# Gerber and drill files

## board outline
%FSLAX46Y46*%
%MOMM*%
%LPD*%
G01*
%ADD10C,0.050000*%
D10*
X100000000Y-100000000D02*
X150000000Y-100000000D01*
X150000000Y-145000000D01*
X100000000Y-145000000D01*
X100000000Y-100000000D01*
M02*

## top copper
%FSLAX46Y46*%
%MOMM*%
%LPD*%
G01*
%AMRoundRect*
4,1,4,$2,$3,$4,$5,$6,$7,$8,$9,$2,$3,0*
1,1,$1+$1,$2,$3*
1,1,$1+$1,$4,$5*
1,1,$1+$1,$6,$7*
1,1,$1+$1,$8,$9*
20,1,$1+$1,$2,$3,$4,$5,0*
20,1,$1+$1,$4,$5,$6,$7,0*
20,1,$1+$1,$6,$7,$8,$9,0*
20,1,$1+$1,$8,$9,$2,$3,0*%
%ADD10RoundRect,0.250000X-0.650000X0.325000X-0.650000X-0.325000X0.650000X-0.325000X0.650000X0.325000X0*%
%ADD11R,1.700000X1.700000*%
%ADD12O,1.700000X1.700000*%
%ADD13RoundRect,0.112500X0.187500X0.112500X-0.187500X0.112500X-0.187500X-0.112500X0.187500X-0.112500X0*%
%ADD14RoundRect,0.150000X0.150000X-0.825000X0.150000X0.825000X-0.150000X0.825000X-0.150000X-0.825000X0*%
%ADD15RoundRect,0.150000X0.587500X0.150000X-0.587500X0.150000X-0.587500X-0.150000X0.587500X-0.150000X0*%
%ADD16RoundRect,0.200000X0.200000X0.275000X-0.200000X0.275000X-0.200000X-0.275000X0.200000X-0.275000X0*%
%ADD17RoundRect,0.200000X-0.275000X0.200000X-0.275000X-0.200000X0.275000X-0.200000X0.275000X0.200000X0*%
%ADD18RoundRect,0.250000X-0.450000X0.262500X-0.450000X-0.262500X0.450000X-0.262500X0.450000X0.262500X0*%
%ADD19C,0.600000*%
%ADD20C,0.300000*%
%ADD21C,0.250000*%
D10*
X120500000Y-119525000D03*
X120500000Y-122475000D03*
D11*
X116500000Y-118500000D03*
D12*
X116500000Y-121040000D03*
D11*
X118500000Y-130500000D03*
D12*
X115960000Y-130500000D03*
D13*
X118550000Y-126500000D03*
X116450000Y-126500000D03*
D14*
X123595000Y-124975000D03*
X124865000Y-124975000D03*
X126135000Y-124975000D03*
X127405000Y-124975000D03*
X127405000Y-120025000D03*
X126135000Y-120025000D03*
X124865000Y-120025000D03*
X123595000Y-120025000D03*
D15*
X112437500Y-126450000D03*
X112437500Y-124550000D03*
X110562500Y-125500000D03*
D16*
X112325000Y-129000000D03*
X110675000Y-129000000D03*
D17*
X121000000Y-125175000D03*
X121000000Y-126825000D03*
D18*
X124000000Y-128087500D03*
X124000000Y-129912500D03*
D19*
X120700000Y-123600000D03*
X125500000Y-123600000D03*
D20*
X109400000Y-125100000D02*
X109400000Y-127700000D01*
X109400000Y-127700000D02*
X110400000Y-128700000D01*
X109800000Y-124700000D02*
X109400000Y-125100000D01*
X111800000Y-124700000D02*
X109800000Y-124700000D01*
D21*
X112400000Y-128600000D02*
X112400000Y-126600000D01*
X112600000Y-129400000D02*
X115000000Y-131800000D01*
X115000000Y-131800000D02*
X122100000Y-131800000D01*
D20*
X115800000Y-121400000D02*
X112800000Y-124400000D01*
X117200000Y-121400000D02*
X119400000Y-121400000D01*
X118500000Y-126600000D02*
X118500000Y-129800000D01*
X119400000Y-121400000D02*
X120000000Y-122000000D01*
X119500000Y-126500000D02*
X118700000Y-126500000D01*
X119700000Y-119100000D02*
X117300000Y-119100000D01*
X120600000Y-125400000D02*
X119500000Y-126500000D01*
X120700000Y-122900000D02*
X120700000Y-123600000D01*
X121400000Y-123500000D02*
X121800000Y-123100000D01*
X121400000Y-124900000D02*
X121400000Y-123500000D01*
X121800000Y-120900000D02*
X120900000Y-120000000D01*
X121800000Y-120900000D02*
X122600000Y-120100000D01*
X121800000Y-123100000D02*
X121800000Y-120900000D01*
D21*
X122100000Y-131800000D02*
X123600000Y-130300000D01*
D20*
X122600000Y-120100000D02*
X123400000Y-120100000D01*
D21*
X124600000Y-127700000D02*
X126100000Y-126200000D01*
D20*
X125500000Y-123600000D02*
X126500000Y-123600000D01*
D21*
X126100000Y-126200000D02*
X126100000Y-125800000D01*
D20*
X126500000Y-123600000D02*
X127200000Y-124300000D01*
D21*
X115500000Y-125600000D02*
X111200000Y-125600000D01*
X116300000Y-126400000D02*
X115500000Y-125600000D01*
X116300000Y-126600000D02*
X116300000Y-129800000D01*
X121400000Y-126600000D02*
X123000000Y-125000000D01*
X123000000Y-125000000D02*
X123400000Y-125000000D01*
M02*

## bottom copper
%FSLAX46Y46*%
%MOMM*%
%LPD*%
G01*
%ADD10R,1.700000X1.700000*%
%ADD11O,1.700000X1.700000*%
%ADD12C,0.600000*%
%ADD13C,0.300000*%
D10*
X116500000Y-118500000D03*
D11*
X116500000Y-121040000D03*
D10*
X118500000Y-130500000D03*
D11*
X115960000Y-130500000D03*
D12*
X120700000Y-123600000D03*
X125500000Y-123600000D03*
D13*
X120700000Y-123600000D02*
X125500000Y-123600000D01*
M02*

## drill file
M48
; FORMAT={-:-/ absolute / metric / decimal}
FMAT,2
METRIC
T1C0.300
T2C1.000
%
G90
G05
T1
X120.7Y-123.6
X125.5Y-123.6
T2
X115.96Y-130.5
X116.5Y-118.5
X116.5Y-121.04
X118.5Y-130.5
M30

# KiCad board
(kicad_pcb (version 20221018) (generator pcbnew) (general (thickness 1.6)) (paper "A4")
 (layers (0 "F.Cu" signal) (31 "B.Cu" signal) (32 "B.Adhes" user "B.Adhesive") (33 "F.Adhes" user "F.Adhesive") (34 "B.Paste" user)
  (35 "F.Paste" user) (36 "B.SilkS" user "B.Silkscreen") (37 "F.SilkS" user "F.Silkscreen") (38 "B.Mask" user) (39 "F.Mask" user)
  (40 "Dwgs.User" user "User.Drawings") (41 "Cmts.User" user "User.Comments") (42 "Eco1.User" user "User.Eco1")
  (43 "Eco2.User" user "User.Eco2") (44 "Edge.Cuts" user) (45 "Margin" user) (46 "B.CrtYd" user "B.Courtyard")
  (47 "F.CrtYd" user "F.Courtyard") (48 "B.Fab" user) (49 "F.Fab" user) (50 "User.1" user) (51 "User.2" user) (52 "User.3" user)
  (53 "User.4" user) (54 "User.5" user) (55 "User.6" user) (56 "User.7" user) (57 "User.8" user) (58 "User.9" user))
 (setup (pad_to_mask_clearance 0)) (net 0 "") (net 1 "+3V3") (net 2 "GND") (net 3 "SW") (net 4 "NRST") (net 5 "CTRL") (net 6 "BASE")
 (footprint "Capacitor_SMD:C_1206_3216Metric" (layer "F.Cu") (at 120.5 121 -90)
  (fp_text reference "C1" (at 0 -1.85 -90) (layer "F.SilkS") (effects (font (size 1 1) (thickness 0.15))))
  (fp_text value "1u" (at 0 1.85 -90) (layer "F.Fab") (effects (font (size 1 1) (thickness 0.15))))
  (pad "1" smd roundrect (at -1.475 0 270) (size 1.15 1.8) (layers "F.Cu" "F.Paste" "F.Mask") (roundrect_rratio 0.217391) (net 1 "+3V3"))
  (pad "2" smd roundrect (at 1.475 0 270) (size 1.15 1.8) (layers "F.Cu" "F.Paste" "F.Mask") (roundrect_rratio 0.217391) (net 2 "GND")))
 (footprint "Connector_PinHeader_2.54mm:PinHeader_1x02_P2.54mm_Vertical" (layer "F.Cu") (at 116.5 118.5)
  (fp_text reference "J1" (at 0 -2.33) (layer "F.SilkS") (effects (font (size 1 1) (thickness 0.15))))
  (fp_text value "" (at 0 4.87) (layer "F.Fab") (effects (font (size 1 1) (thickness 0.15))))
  (pad "1" thru_hole rect (at 0 0) (size 1.7 1.7) (drill 1) (layers "*.Cu" "*.Mask") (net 1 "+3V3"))
  (pad "2" thru_hole oval (at 0 2.54) (size 1.7 1.7) (drill 1) (layers "*.Cu" "*.Mask") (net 2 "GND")))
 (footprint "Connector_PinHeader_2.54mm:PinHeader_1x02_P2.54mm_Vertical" (layer "F.Cu") (at 118.5 130.5 -90)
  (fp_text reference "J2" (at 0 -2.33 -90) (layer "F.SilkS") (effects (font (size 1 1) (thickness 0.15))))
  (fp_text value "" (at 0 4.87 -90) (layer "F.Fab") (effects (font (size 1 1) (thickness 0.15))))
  (pad "1" thru_hole rect (at 0 0 270) (size 1.7 1.7) (drill 1) (layers "*.Cu" "*.Mask") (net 1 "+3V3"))
  (pad "2" thru_hole oval (at 0 2.54 270) (size 1.7 1.7) (drill 1) (layers "*.Cu" "*.Mask") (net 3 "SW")))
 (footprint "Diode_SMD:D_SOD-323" (layer "F.Cu") (at 117.5 126.5 180)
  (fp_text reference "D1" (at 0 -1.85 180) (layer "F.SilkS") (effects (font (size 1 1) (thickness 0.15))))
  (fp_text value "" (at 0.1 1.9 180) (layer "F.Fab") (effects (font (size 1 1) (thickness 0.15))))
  (pad "1" smd roundrect (at -1.05 0 180) (size 0.6 0.45) (layers "F.Cu" "F.Paste" "F.Mask") (roundrect_rratio 0.25) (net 1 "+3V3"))
  (pad "2" smd roundrect (at 1.05 0 180) (size 0.6 0.45) (layers "F.Cu" "F.Paste" "F.Mask") (roundrect_rratio 0.25) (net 3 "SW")))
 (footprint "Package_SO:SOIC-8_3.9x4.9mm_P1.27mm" (layer "F.Cu") (at 125.5 122.5 90)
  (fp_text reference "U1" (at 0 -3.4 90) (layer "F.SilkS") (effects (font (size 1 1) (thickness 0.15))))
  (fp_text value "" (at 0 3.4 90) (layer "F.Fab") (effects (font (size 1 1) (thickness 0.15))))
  (pad "1" smd roundrect (at -2.475 -1.905 90) (size 1.95 0.6) (layers "F.Cu" "F.Paste" "F.Mask") (roundrect_rratio 0.25) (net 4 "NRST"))
  (pad "2" smd roundrect (at -2.475 -0.635 90) (size 1.95 0.6) (layers "F.Cu" "F.Paste" "F.Mask") (roundrect_rratio 0.25))
  (pad "3" smd roundrect (at -2.475 0.635 90) (size 1.95 0.6) (layers "F.Cu" "F.Paste" "F.Mask") (roundrect_rratio 0.25) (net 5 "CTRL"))
  (pad "4" smd roundrect (at -2.475 1.905 90) (size 1.95 0.6) (layers "F.Cu" "F.Paste" "F.Mask") (roundrect_rratio 0.25) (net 2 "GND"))
  (pad "5" smd roundrect (at 2.475 1.905 90) (size 1.95 0.6) (layers "F.Cu" "F.Paste" "F.Mask") (roundrect_rratio 0.25))
  (pad "6" smd roundrect (at 2.475 0.635 90) (size 1.95 0.6) (layers "F.Cu" "F.Paste" "F.Mask") (roundrect_rratio 0.25))
  (pad "7" smd roundrect (at 2.475 -0.635 90) (size 1.95 0.6) (layers "F.Cu" "F.Paste" "F.Mask") (roundrect_rratio 0.25))
  (pad "8" smd roundrect (at 2.475 -1.905 90) (size 1.95 0.6) (layers "F.Cu" "F.Paste" "F.Mask") (roundrect_rratio 0.25) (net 1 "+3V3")))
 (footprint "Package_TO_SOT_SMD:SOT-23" (layer "F.Cu") (at 111.5 125.5 180)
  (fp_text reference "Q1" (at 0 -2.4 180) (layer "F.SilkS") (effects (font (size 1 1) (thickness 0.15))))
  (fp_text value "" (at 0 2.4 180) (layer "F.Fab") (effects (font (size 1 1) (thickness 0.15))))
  (pad "1" smd roundrect (at -0.9375 -0.95 180) (size 1.475 0.6) (layers "F.Cu" "F.Paste" "F.Mask") (roundrect_rratio 0.25) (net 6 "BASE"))
  (pad "2" smd roundrect (at -0.9375 0.95 180) (size 1.475 0.6) (layers "F.Cu" "F.Paste" "F.Mask") (roundrect_rratio 0.25) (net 2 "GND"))
  (pad "3" smd roundrect (at 0.9375 0 180) (size 1.475 0.6) (layers "F.Cu" "F.Paste" "F.Mask") (roundrect_rratio 0.25) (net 3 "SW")))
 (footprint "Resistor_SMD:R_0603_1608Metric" (layer "F.Cu") (at 111.5 129 180)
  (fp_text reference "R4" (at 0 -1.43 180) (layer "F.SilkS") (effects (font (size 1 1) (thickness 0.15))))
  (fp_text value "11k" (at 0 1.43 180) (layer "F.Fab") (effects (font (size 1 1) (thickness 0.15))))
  (pad "1" smd roundrect (at -0.825 0 180) (size 0.8 0.95) (layers "F.Cu" "F.Paste" "F.Mask") (roundrect_rratio 0.25) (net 6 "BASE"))
  (pad "2" smd roundrect (at 0.825 0 180) (size 0.8 0.95) (layers "F.Cu" "F.Paste" "F.Mask") (roundrect_rratio 0.25) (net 2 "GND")))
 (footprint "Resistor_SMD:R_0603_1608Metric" (layer "F.Cu") (at 121 126 -90)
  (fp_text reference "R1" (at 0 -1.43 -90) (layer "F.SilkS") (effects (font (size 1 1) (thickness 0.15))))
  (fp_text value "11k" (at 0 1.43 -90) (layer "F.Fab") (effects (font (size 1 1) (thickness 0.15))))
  (pad "1" smd roundrect (at -0.825 0 270) (size 0.8 0.95) (layers "F.Cu" "F.Paste" "F.Mask") (roundrect_rratio 0.25) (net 1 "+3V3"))
  (pad "2" smd roundrect (at 0.825 0 270) (size 0.8 0.95) (layers "F.Cu" "F.Paste" "F.Mask") (roundrect_rratio 0.25) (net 4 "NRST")))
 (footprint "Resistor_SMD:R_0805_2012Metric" (layer "F.Cu") (at 124 129 -90)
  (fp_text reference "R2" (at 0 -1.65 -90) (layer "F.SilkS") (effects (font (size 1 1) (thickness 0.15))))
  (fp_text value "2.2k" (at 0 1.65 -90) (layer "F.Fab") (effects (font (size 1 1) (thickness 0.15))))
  (pad "1" smd roundrect (at -0.9125 0 270) (size 1.025 1.4) (layers "F.Cu" "F.Paste" "F.Mask") (roundrect_rratio 0.243902) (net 5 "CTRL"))
  (pad "2" smd roundrect (at 0.9125 0 270) (size 1.025 1.4) (layers "F.Cu" "F.Paste" "F.Mask") (roundrect_rratio 0.243902) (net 6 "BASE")))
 (gr_rect (start 100 100) (end 150 145) (stroke (width 0.05) (type default)) (fill none) (layer "Edge.Cuts"))
 (segment (start 109.4 125.1) (end 109.4 127.7) (width 0.3) (layer "F.Cu") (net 2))
 (segment (start 109.4 127.7) (end 110.4 128.7) (width 0.3) (layer "F.Cu") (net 2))
 (segment (start 109.8 124.7) (end 109.4 125.1) (width 0.3) (layer "F.Cu") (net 2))
 (segment (start 111.8 124.7) (end 109.8 124.7) (width 0.3) (layer "F.Cu") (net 2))
 (segment (start 112.4 128.6) (end 112.4 126.6) (width 0.25) (layer "F.Cu") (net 6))
 (segment (start 112.6 129.4) (end 115 131.8) (width 0.25) (layer "F.Cu") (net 6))
 (segment (start 115 131.8) (end 122.1 131.8) (width 0.25) (layer "F.Cu") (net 6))
 (segment (start 115.8 121.4) (end 112.8 124.4) (width 0.3) (layer "F.Cu") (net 2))
 (segment (start 117.2 121.4) (end 119.4 121.4) (width 0.3) (layer "F.Cu") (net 2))
 (segment (start 118.5 126.6) (end 118.5 129.8) (width 0.3) (layer "F.Cu") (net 1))
 (segment (start 119.4 121.4) (end 120 122) (width 0.3) (layer "F.Cu") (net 2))
 (segment (start 119.5 126.5) (end 118.7 126.5) (width 0.3) (layer "F.Cu") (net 1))
 (segment (start 119.7 119.1) (end 117.3 119.1) (width 0.3) (layer "F.Cu") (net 1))
 (segment (start 120.6 125.4) (end 119.5 126.5) (width 0.3) (layer "F.Cu") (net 1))
 (segment (start 120.7 122.9) (end 120.7 123.6) (width 0.3) (layer "F.Cu") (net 2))
 (segment (start 121.4 123.5) (end 121.8 123.1) (width 0.3) (layer "F.Cu") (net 1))
 (segment (start 121.4 124.9) (end 121.4 123.5) (width 0.3) (layer "F.Cu") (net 1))
 (segment (start 121.8 120.9) (end 120.9 120) (width 0.3) (layer "F.Cu") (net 1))
 (segment (start 121.8 120.9) (end 122.6 120.1) (width 0.3) (layer "F.Cu") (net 1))
 (segment (start 121.8 123.1) (end 121.8 120.9) (width 0.3) (layer "F.Cu") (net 1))
 (segment (start 122.1 131.8) (end 123.6 130.3) (width 0.25) (layer "F.Cu") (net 6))
 (segment (start 122.6 120.1) (end 123.4 120.1) (width 0.3) (layer "F.Cu") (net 1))
 (segment (start 124.6 127.7) (end 126.1 126.2) (width 0.25) (layer "F.Cu") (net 5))
 (segment (start 125.5 123.6) (end 126.5 123.6) (width 0.3) (layer "F.Cu") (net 2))
 (segment (start 126.1 126.2) (end 126.1 125.8) (width 0.25) (layer "F.Cu") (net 5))
 (segment (start 126.5 123.6) (end 127.2 124.3) (width 0.3) (layer "F.Cu") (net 2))
 (via (at 120.7 123.6) (size 0.6) (drill 0.3) (layers "F.Cu" "B.Cu") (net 2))
 (via (at 125.5 123.6) (size 0.6) (drill 0.3) (layers "F.Cu" "B.Cu") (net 2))
 (segment (start 115.5 125.6) (end 111.2 125.6) (width 0.25) (layer "F.Cu") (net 3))
 (segment (start 116.3 126.4) (end 115.5 125.6) (width 0.25) (layer "F.Cu") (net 3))
 (segment (start 116.3 126.6) (end 116.3 129.8) (width 0.25) (layer "F.Cu") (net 3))
 (segment (start 120.7 123.6) (end 125.5 123.6) (width 0.3) (layer "B.Cu") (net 2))
 (segment (start 121.4 126.6) (end 123 125) (width 0.25) (layer "F.Cu") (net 4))
 (segment (start 123 125) (end 123.4 125) (width 0.25) (layer "F.Cu") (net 4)))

